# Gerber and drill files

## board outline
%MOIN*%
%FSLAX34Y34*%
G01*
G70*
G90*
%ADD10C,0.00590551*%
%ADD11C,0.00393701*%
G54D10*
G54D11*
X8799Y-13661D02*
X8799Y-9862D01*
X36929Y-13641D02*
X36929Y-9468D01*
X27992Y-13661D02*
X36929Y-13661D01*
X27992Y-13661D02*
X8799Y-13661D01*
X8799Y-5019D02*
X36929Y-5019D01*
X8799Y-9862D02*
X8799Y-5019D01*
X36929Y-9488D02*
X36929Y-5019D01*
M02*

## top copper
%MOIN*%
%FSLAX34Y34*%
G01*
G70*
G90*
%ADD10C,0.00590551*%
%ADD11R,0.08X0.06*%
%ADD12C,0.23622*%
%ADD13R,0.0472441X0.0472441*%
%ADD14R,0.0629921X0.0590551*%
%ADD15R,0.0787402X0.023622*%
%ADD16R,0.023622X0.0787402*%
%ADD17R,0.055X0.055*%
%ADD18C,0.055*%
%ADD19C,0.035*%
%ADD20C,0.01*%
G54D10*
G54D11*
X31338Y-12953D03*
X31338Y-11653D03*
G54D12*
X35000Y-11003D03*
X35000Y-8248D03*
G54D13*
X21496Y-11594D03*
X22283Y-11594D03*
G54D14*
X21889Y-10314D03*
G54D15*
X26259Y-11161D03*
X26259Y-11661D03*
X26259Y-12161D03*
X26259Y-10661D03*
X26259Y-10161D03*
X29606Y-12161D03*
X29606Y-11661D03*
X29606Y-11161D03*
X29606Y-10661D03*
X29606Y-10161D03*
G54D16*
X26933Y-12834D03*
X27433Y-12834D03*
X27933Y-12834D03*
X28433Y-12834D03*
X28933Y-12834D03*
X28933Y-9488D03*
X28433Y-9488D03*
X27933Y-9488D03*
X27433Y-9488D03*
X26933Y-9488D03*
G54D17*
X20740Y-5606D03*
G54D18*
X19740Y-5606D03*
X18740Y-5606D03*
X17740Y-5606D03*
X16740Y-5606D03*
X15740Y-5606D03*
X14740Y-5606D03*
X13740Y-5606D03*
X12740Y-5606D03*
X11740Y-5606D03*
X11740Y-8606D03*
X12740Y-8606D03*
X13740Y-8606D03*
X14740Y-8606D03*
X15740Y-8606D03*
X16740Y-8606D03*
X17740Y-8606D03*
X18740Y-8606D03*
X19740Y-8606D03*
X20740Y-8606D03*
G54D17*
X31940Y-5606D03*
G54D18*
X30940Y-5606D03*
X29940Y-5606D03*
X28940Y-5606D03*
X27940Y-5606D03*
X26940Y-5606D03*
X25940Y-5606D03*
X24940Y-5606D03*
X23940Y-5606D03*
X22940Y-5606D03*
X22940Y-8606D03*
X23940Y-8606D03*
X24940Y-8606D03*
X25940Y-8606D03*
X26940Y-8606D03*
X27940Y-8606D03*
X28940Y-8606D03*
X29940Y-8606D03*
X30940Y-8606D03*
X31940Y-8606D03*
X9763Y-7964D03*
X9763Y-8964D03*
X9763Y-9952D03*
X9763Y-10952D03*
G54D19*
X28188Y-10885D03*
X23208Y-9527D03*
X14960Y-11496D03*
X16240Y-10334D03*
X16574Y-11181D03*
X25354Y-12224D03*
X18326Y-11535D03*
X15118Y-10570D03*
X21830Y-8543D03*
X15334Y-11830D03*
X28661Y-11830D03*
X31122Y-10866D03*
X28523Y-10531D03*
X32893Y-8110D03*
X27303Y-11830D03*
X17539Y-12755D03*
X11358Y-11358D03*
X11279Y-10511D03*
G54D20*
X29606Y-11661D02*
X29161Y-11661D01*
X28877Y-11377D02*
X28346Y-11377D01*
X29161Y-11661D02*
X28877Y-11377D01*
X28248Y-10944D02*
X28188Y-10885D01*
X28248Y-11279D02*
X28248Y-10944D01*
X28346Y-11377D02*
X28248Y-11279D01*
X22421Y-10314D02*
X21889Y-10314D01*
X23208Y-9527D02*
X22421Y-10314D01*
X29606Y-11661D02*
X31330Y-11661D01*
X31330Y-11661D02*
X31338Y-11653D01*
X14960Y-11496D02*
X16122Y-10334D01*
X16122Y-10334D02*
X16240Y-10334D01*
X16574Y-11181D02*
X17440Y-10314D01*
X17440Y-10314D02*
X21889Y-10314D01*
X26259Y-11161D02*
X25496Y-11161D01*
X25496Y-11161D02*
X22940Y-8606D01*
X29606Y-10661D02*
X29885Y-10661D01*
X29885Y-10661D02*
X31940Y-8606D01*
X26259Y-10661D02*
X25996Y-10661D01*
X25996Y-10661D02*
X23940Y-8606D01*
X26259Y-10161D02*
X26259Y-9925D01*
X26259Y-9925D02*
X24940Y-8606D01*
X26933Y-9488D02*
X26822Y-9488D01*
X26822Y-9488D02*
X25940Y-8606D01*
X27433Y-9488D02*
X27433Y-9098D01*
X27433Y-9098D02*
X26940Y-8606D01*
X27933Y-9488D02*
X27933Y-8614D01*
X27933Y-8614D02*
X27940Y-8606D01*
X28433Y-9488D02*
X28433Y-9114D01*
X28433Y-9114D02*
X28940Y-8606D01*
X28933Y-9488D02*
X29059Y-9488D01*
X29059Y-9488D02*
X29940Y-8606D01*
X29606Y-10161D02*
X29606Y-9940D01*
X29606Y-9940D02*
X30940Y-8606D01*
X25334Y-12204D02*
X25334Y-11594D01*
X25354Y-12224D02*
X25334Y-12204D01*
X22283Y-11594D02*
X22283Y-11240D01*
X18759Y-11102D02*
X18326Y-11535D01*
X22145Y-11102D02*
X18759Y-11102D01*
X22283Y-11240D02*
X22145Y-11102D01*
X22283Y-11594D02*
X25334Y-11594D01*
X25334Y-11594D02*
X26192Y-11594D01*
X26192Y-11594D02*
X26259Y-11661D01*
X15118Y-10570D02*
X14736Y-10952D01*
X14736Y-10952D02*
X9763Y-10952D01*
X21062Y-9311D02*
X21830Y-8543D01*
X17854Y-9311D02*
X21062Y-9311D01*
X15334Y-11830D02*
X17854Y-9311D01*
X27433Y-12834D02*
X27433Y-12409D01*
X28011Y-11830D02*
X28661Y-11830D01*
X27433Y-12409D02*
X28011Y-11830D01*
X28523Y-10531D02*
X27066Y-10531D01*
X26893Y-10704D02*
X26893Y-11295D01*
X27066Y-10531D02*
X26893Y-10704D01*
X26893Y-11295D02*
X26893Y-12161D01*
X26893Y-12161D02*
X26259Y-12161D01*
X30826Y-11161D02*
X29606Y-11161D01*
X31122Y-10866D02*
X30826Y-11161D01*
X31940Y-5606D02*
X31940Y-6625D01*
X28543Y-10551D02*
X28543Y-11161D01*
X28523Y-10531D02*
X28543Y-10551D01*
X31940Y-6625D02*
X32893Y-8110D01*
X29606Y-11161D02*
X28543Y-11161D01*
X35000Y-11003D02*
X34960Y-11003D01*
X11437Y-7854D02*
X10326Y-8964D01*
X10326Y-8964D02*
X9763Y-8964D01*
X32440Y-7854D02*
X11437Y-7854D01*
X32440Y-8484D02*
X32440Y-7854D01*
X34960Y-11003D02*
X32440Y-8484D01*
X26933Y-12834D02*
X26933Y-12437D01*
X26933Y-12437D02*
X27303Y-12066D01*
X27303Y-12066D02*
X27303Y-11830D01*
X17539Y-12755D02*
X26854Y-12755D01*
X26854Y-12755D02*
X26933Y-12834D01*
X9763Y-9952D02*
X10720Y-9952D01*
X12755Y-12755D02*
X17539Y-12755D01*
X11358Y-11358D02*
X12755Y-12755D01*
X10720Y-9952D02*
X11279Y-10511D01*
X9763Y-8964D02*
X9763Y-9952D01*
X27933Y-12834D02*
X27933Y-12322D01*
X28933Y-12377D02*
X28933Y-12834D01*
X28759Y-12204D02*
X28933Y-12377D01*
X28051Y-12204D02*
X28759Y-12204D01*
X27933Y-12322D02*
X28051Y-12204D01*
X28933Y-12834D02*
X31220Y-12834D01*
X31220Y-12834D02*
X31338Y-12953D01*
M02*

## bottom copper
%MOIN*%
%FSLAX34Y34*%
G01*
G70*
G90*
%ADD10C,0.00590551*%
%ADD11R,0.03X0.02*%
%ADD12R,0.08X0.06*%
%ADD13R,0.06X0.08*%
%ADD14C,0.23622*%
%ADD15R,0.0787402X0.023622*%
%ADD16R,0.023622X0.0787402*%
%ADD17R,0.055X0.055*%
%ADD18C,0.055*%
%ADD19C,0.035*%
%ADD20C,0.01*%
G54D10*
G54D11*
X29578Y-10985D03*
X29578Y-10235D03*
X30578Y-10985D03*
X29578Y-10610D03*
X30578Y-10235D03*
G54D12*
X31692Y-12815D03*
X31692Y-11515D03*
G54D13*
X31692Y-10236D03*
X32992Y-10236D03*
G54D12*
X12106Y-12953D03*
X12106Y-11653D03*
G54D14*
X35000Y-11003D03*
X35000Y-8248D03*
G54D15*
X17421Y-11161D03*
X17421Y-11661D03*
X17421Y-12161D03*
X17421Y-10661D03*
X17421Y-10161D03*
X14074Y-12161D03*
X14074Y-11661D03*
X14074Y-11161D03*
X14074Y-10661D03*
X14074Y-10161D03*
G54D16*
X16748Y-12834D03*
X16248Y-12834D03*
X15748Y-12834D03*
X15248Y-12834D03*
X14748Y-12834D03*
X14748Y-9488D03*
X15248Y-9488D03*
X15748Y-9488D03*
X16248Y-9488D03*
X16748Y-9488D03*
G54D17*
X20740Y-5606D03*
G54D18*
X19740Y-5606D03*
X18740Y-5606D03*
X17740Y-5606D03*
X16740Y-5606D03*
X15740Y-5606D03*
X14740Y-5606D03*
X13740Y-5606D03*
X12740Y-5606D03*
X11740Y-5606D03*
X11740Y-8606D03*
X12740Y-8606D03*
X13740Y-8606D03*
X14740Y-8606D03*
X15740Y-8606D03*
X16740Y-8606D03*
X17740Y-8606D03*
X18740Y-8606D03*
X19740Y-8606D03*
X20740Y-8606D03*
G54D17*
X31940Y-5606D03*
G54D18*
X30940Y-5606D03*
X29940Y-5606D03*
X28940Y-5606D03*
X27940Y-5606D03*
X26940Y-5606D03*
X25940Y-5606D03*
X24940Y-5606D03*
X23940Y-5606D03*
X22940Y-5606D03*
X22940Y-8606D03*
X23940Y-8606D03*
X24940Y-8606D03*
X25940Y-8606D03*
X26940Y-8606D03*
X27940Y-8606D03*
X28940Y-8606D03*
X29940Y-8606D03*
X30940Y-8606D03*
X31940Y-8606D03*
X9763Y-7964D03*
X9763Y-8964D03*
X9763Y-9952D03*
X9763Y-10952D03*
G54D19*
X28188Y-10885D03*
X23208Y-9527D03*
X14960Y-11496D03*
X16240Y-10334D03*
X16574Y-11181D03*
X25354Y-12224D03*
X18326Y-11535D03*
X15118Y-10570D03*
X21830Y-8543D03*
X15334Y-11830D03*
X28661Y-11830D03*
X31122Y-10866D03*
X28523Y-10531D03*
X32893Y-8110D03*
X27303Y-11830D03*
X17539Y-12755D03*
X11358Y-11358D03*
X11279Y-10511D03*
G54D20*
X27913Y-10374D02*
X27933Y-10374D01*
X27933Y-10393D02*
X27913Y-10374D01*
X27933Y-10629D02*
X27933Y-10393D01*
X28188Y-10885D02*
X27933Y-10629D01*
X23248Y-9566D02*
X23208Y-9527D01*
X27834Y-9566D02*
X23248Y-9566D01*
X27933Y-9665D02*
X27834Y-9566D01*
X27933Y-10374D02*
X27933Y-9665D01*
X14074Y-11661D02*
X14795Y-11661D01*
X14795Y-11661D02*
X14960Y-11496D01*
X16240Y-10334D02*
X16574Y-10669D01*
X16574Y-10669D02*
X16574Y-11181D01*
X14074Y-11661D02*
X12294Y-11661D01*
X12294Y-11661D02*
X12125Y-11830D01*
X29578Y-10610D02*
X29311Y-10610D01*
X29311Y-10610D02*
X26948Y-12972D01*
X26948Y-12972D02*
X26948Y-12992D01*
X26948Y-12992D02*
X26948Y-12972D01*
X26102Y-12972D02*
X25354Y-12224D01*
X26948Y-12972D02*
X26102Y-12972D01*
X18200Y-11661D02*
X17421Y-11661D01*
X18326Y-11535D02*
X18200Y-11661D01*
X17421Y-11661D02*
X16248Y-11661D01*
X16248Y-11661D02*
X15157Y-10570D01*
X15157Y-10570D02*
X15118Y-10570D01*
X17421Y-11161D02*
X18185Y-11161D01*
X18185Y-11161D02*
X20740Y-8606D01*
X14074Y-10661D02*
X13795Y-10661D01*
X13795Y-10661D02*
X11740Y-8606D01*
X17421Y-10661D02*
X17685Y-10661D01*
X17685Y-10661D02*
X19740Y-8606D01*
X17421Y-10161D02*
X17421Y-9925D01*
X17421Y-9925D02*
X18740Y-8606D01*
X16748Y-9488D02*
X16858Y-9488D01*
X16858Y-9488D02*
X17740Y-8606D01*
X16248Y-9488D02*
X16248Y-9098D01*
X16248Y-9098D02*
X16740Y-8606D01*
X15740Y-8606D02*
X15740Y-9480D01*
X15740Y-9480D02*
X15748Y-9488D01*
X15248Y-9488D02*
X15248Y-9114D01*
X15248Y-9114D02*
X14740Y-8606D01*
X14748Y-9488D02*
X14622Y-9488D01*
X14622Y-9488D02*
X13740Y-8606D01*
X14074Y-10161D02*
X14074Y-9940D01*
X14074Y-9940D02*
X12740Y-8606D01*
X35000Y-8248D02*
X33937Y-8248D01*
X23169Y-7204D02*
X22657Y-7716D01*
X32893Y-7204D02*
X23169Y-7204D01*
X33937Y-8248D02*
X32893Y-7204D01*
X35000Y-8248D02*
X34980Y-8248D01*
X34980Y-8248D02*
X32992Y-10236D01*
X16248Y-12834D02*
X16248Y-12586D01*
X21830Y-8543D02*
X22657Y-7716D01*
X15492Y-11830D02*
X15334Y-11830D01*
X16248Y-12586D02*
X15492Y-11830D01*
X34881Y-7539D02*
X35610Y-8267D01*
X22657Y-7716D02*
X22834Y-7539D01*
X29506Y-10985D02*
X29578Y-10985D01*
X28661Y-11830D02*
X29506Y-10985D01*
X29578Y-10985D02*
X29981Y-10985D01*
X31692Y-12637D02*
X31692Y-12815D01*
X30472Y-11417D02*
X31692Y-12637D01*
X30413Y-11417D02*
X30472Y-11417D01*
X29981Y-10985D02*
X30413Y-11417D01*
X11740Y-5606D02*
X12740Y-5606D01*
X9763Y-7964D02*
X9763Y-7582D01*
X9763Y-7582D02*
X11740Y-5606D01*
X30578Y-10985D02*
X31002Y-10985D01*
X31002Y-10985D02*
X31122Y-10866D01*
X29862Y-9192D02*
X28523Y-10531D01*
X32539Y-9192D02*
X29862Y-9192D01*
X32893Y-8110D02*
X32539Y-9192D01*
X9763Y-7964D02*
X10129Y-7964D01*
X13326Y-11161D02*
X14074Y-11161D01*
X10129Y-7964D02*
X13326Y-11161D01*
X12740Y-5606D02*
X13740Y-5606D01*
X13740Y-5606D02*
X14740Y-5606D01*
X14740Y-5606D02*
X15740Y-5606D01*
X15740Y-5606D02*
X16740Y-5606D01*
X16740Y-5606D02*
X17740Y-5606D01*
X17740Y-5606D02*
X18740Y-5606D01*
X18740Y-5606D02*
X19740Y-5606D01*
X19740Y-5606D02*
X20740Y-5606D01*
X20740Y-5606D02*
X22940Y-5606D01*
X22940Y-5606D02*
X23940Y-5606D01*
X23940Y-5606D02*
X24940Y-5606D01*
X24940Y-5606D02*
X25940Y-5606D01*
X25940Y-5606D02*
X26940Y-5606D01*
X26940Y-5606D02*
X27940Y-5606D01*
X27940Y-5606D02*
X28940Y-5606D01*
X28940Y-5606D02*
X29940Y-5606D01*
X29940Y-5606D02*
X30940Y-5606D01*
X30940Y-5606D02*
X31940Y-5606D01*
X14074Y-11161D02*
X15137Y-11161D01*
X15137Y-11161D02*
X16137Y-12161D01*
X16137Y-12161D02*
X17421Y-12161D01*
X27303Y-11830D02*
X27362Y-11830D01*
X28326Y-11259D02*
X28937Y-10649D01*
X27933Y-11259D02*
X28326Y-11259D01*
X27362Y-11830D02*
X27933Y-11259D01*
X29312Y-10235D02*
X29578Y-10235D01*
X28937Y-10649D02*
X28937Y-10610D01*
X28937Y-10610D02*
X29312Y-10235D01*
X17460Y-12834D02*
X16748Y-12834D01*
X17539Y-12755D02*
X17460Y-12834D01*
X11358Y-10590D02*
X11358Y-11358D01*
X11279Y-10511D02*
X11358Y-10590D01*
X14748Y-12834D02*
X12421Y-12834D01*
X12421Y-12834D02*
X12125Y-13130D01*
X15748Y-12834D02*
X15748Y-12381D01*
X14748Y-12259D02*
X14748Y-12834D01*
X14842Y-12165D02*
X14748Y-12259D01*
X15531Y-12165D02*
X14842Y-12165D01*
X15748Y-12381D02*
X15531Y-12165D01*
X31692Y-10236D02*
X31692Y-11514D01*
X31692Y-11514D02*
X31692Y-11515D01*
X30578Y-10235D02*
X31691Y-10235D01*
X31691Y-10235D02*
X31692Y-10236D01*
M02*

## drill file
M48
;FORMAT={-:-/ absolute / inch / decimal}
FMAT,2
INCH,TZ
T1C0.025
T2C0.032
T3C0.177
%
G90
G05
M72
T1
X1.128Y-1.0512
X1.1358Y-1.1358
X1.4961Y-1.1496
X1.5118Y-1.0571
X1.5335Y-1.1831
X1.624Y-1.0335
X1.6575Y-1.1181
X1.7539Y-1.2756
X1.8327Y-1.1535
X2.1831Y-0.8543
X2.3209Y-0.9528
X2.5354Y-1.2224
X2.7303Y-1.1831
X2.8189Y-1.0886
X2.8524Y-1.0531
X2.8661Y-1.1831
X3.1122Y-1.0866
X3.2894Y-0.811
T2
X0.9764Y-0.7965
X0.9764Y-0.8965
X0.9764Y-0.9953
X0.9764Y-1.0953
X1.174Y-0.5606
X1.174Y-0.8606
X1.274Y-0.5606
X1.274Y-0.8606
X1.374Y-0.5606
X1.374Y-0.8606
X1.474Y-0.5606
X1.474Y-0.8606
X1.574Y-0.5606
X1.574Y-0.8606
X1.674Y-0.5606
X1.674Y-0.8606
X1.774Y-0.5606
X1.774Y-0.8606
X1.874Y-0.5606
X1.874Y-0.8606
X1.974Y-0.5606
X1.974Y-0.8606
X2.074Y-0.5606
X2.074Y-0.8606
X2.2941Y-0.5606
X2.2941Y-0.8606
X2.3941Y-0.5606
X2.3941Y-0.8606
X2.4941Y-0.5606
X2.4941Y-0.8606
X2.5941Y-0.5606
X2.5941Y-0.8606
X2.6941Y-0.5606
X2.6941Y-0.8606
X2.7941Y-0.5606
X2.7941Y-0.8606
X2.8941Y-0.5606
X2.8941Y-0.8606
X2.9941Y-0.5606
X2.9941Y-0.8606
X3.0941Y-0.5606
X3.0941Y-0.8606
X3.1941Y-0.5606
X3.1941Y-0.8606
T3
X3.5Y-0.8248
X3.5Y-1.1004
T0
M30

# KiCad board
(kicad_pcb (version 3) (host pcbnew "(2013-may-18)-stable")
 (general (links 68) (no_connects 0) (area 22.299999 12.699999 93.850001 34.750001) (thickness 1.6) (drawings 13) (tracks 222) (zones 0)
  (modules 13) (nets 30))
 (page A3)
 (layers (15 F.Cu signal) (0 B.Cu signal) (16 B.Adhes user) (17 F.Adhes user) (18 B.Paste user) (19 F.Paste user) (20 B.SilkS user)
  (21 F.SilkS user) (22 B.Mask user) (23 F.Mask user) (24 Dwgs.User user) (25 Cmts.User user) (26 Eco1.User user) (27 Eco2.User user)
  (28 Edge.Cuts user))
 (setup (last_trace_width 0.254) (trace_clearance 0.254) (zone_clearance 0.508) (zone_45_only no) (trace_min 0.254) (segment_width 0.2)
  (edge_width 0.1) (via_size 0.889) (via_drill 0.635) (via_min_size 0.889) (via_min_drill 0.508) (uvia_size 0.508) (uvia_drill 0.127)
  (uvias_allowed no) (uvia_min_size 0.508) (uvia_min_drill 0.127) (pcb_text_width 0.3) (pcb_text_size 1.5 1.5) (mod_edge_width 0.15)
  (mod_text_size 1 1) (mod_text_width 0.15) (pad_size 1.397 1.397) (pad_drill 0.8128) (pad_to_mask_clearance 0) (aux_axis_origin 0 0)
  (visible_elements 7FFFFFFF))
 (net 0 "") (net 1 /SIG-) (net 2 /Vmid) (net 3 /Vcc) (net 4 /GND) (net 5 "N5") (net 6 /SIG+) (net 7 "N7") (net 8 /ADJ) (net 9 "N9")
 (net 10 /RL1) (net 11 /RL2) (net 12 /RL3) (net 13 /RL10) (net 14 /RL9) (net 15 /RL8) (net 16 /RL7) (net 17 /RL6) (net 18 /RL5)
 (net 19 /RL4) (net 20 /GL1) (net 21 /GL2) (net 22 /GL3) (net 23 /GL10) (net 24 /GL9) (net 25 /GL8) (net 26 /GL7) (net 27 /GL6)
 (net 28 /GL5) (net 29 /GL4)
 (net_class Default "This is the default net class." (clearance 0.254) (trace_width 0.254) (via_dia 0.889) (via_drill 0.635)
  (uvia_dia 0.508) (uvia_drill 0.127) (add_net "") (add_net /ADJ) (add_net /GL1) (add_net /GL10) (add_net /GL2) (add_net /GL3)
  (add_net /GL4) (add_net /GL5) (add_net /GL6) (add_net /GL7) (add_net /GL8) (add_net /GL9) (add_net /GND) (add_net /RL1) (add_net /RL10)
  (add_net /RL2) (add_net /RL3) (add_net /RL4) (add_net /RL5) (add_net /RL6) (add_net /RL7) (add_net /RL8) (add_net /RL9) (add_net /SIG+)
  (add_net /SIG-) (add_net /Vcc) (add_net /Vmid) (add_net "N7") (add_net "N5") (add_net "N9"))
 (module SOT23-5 (layer B.Cu) (at 76.4 26.95 90)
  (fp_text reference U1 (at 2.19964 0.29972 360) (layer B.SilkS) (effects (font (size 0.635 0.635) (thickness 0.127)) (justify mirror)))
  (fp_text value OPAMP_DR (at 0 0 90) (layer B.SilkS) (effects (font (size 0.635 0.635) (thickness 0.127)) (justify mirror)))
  (pad 1 smd rect (at -0.9525 -1.27 90) (size 0.508 0.762) (layers B.Cu B.Paste B.Mask) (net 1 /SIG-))
  (pad 3 smd rect (at 0.9525 -1.27 90) (size 0.508 0.762) (layers B.Cu B.Paste B.Mask) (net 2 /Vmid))
  (pad 5 smd rect (at -0.9525 1.27 90) (size 0.508 0.762) (layers B.Cu B.Paste B.Mask) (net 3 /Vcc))
  (pad 2 smd rect (at 0 -1.27 90) (size 0.508 0.762) (layers B.Cu B.Paste B.Mask) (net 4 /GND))
  (pad 4 smd rect (at 0.9525 1.27 90) (size 0.508 0.762) (layers B.Cu B.Paste B.Mask) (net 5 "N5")))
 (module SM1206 (layer B.Cu) (at 80.5 30.9 90)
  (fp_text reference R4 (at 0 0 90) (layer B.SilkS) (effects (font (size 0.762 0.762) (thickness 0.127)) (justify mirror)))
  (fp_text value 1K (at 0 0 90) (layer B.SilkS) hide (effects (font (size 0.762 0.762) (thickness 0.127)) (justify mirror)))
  (pad 1 smd rect (at -1.651 0 90) (size 1.524 2.032) (layers B.Cu B.Paste B.Mask) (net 1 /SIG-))
  (pad 2 smd rect (at 1.651 0 90) (size 1.524 2.032) (layers B.Cu B.Paste B.Mask) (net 5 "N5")))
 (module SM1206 (layer B.Cu) (at 82.15 26)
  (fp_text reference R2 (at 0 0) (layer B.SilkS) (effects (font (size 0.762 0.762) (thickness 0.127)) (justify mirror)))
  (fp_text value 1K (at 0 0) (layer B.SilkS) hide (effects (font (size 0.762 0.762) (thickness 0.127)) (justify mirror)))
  (pad 1 smd rect (at -1.651 0) (size 1.524 2.032) (layers B.Cu B.Paste B.Mask) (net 5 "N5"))
  (pad 2 smd rect (at 1.651 0) (size 1.524 2.032) (layers B.Cu B.Paste B.Mask) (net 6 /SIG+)))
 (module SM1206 (layer B.Cu) (at 30.75 31.25 90)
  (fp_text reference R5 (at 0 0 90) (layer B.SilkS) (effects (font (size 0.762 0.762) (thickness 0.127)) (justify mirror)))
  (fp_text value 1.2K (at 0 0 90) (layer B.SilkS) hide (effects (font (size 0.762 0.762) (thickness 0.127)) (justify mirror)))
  (pad 1 smd rect (at -1.651 0 90) (size 1.524 2.032) (layers B.Cu B.Paste B.Mask) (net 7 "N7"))
  (pad 2 smd rect (at 1.651 0 90) (size 1.524 2.032) (layers B.Cu B.Paste B.Mask) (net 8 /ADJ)))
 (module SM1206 (layer F.Cu) (at 79.6 31.25 90)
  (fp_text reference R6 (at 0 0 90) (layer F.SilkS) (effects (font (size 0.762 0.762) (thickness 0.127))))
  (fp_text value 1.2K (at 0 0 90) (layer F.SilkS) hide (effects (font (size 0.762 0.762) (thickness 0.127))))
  (pad 1 smd rect (at -1.651 0 90) (size 1.524 2.032) (layers F.Cu F.Paste F.Mask) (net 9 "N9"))
  (pad 2 smd rect (at 1.651 0 90) (size 1.524 2.032) (layers F.Cu F.Paste F.Mask) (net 8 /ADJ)))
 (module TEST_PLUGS (layer F.Cu) (at 88.9 27.95 90)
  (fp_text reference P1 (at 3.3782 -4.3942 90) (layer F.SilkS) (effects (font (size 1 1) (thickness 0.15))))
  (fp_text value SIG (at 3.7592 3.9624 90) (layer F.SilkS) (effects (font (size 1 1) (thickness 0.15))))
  (pad 1 thru_hole circle (at 0 0 90) (size 6 6) (drill 4.5) (layers *.Cu *.Mask F.SilkS) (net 2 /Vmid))
  (pad 2 thru_hole circle (at 7 0 90) (size 6 6) (drill 4.5) (layers *.Cu *.Mask F.SilkS) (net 6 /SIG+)))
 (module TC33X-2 (layer F.Cu) (at 55.6 27.65)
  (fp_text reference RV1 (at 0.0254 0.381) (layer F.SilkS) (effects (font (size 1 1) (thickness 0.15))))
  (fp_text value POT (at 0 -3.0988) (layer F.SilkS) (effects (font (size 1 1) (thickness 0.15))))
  (pad 1 smd rect (at -1 1.8) (size 1.2 1.2) (layers F.Cu F.Paste F.Mask))
  (pad 3 smd rect (at 1 1.8) (size 1.2 1.2) (layers F.Cu F.Paste F.Mask) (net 4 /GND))
  (pad 2 smd rect (at 0 -1.45) (size 1.6 1.5) (layers F.Cu F.Paste F.Mask) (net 8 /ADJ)))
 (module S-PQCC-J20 (layer B.Cu) (at 40 28.35 90)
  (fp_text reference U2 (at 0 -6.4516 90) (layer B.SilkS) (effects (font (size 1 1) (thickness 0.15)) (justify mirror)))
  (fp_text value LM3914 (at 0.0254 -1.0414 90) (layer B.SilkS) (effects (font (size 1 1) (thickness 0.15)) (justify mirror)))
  (pad 1 smd rect (at 0 4.25 90) (size 0.6 2) (layers B.Cu B.Paste B.Mask) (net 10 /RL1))
  (pad 2 smd rect (at -1.27 4.25 90) (size 0.6 2) (layers B.Cu B.Paste B.Mask) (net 4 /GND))
  (pad 3 smd rect (at -2.54 4.25 90) (size 0.6 2) (layers B.Cu B.Paste B.Mask) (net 3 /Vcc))
  (pad 20 smd rect (at 1.27 4.25 90) (size 0.6 2) (layers B.Cu B.Paste B.Mask) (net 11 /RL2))
  (pad 19 smd rect (at 2.54 4.25 90) (size 0.6 2) (layers B.Cu B.Paste B.Mask) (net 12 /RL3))
  (pad 9 smd rect (at -2.54 -4.25 90) (size 0.6 2) (layers B.Cu B.Paste B.Mask))
  (pad 10 smd rect (at -1.27 -4.25 90) (size 0.6 2) (layers B.Cu B.Paste B.Mask) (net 8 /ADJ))
  (pad 11 smd rect (at 0 -4.25 90) (size 0.6 2) (layers B.Cu B.Paste B.Mask) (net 3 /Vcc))
  (pad 12 smd rect (at 1.27 -4.25 90) (size 0.6 2) (layers B.Cu B.Paste B.Mask) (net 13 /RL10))
  (pad 13 smd rect (at 2.54 -4.25 90) (size 0.6 2) (layers B.Cu B.Paste B.Mask) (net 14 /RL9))
  (pad 4 smd rect (at -4.25 2.54 90) (size 2 0.6) (layers B.Cu B.Paste B.Mask) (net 2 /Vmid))
  (pad 5 smd rect (at -4.25 1.27 90) (size 2 0.6) (layers B.Cu B.Paste B.Mask) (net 6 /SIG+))
  (pad 6 smd rect (at -4.25 0 90) (size 2 0.6) (layers B.Cu B.Paste B.Mask) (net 7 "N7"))
  (pad 7 smd rect (at -4.25 -1.27 90) (size 2 0.6) (layers B.Cu B.Paste B.Mask))
  (pad 8 smd rect (at -4.25 -2.54 90) (size 2 0.6) (layers B.Cu B.Paste B.Mask) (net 7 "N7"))
  (pad 14 smd rect (at 4.25 -2.54 90) (size 2 0.6) (layers B.Cu B.Paste B.Mask) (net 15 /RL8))
  (pad 15 smd rect (at 4.25 -1.27 90) (size 2 0.6) (layers B.Cu B.Paste B.Mask) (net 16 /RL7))
  (pad 16 smd rect (at 4.25 0 90) (size 2 0.6) (layers B.Cu B.Paste B.Mask) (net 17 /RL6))
  (pad 17 smd rect (at 4.25 1.27 90) (size 2 0.6) (layers B.Cu B.Paste B.Mask) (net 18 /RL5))
  (pad 18 smd rect (at 4.25 2.54 90) (size 2 0.6) (layers B.Cu B.Paste B.Mask) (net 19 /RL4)))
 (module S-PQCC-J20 (layer F.Cu) (at 70.95 28.35 90)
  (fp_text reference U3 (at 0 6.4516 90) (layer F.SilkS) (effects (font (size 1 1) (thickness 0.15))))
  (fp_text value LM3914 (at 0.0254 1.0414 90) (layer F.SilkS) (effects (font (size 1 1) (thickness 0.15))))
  (pad 1 smd rect (at 0 -4.25 90) (size 0.6 2) (layers F.Cu F.Paste F.Mask) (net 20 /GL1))
  (pad 2 smd rect (at -1.27 -4.25 90) (size 0.6 2) (layers F.Cu F.Paste F.Mask) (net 4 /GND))
  (pad 3 smd rect (at -2.54 -4.25 90) (size 0.6 2) (layers F.Cu F.Paste F.Mask) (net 3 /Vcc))
  (pad 20 smd rect (at 1.27 -4.25 90) (size 0.6 2) (layers F.Cu F.Paste F.Mask) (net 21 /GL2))
  (pad 19 smd rect (at 2.54 -4.25 90) (size 0.6 2) (layers F.Cu F.Paste F.Mask) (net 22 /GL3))
  (pad 9 smd rect (at -2.54 4.25 90) (size 0.6 2) (layers F.Cu F.Paste F.Mask))
  (pad 10 smd rect (at -1.27 4.25 90) (size 0.6 2) (layers F.Cu F.Paste F.Mask) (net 8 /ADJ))
  (pad 11 smd rect (at 0 4.25 90) (size 0.6 2) (layers F.Cu F.Paste F.Mask) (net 3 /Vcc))
  (pad 12 smd rect (at 1.27 4.25 90) (size 0.6 2) (layers F.Cu F.Paste F.Mask) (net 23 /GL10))
  (pad 13 smd rect (at 2.54 4.25 90) (size 0.6 2) (layers F.Cu F.Paste F.Mask) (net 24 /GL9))
  (pad 4 smd rect (at -4.25 -2.54 90) (size 2 0.6) (layers F.Cu F.Paste F.Mask) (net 2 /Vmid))
  (pad 5 smd rect (at -4.25 -1.27 90) (size 2 0.6) (layers F.Cu F.Paste F.Mask) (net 1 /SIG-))
  (pad 6 smd rect (at -4.25 0 90) (size 2 0.6) (layers F.Cu F.Paste F.Mask) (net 9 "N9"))
  (pad 7 smd rect (at -4.25 1.27 90) (size 2 0.6) (layers F.Cu F.Paste F.Mask))
  (pad 8 smd rect (at -4.25 2.54 90) (size 2 0.6) (layers F.Cu F.Paste F.Mask) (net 9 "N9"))
  (pad 14 smd rect (at 4.25 2.54 90) (size 2 0.6) (layers F.Cu F.Paste F.Mask) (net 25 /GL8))
  (pad 15 smd rect (at 4.25 1.27 90) (size 2 0.6) (layers F.Cu F.Paste F.Mask) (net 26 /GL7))
  (pad 16 smd rect (at 4.25 0 90) (size 2 0.6) (layers F.Cu F.Paste F.Mask) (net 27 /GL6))
  (pad 17 smd rect (at 4.25 -1.27 90) (size 2 0.6) (layers F.Cu F.Paste F.Mask) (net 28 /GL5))
  (pad 18 smd rect (at 4.25 -2.54 90) (size 2 0.6) (layers F.Cu F.Paste F.Mask) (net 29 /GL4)))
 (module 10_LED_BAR (layer F.Cu) (at 41.25 18.05 180)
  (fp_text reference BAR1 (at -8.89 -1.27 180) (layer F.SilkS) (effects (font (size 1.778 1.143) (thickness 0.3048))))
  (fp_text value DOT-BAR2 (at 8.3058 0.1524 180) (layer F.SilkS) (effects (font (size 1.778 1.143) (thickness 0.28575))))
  (pad 1 thru_hole rect (at -11.43 3.81 180) (size 1.397 1.397) (drill 0.8128) (layers *.Cu *.Mask F.SilkS) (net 3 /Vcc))
  (pad 2 thru_hole circle (at -8.89 3.81 180) (size 1.397 1.397) (drill 0.8128) (layers *.Cu *.Mask F.SilkS) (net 3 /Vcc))
  (pad 3 thru_hole circle (at -6.35 3.81 180) (size 1.397 1.397) (drill 0.8128) (layers *.Cu *.Mask F.SilkS) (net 3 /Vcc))
  (pad 4 thru_hole circle (at -3.81 3.81 180) (size 1.397 1.397) (drill 0.8128) (layers *.Cu *.Mask F.SilkS) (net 3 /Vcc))
  (pad 5 thru_hole circle (at -1.27 3.81 180) (size 1.397 1.397) (drill 0.8128) (layers *.Cu *.Mask F.SilkS) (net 3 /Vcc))
  (pad 6 thru_hole circle (at 1.27 3.81 180) (size 1.397 1.397) (drill 0.8128) (layers *.Cu *.Mask F.SilkS) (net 3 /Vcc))
  (pad 7 thru_hole circle (at 3.81 3.81 180) (size 1.397 1.397) (drill 0.8128) (layers *.Cu *.Mask F.SilkS) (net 3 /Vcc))
  (pad 8 thru_hole circle (at 6.35 3.81 180) (size 1.397 1.397) (drill 0.8128) (layers *.Cu *.Mask F.SilkS) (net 3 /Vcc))
  (pad 9 thru_hole circle (at 8.89 3.81 180) (size 1.397 1.397) (drill 0.8128) (layers *.Cu *.Mask F.SilkS) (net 3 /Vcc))
  (pad 10 thru_hole circle (at 11.43 3.81 180) (size 1.397 1.397) (drill 0.8128) (layers *.Cu *.Mask F.SilkS) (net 3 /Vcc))
  (pad 11 thru_hole circle (at 11.43 -3.81 180) (size 1.397 1.397) (drill 0.8128) (layers *.Cu *.Mask F.SilkS) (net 13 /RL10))
  (pad 12 thru_hole circle (at 8.89 -3.81 180) (size 1.397 1.397) (drill 0.8128) (layers *.Cu *.Mask F.SilkS) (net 14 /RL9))
  (pad 13 thru_hole circle (at 6.35 -3.81 180) (size 1.397 1.397) (drill 0.8128) (layers *.Cu *.Mask F.SilkS) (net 15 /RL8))
  (pad 14 thru_hole circle (at 3.81 -3.81 180) (size 1.397 1.397) (drill 0.8128) (layers *.Cu *.Mask F.SilkS) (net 16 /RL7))
  (pad 15 thru_hole circle (at 1.27 -3.81 180) (size 1.397 1.397) (drill 0.8128) (layers *.Cu *.Mask F.SilkS) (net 17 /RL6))
  (pad 16 thru_hole circle (at -1.27 -3.81 180) (size 1.397 1.397) (drill 0.8128) (layers *.Cu *.Mask F.SilkS) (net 18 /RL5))
  (pad 17 thru_hole circle (at -3.81 -3.81 180) (size 1.397 1.397) (drill 0.8128) (layers *.Cu *.Mask F.SilkS) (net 19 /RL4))
  (pad 18 thru_hole circle (at -6.35 -3.81 180) (size 1.397 1.397) (drill 0.8128) (layers *.Cu *.Mask F.SilkS) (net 12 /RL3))
  (pad 19 thru_hole circle (at -8.89 -3.81 180) (size 1.397 1.397) (drill 0.8128) (layers *.Cu *.Mask F.SilkS) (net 11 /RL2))
  (pad 20 thru_hole circle (at -11.43 -3.81 180) (size 1.397 1.397) (drill 0.8128) (layers *.Cu *.Mask F.SilkS) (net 10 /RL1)))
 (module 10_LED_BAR (layer F.Cu) (at 69.7 18.05 180)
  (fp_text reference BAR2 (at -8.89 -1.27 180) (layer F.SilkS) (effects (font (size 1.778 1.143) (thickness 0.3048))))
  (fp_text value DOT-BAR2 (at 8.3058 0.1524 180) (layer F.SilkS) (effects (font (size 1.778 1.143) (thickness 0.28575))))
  (pad 1 thru_hole rect (at -11.43 3.81 180) (size 1.397 1.397) (drill 0.8128) (layers *.Cu *.Mask F.SilkS) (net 3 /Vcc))
  (pad 2 thru_hole circle (at -8.89 3.81 180) (size 1.397 1.397) (drill 0.8128) (layers *.Cu *.Mask F.SilkS) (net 3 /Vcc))
  (pad 3 thru_hole circle (at -6.35 3.81 180) (size 1.397 1.397) (drill 0.8128) (layers *.Cu *.Mask F.SilkS) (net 3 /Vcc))
  (pad 4 thru_hole circle (at -3.81 3.81 180) (size 1.397 1.397) (drill 0.8128) (layers *.Cu *.Mask F.SilkS) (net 3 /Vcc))
  (pad 5 thru_hole circle (at -1.27 3.81 180) (size 1.397 1.397) (drill 0.8128) (layers *.Cu *.Mask F.SilkS) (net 3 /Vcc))
  (pad 6 thru_hole circle (at 1.27 3.81 180) (size 1.397 1.397) (drill 0.8128) (layers *.Cu *.Mask F.SilkS) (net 3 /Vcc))
  (pad 7 thru_hole circle (at 3.81 3.81 180) (size 1.397 1.397) (drill 0.8128) (layers *.Cu *.Mask F.SilkS) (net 3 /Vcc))
  (pad 8 thru_hole circle (at 6.35 3.81 180) (size 1.397 1.397) (drill 0.8128) (layers *.Cu *.Mask F.SilkS) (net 3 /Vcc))
  (pad 9 thru_hole circle (at 8.89 3.81 180) (size 1.397 1.397) (drill 0.8128) (layers *.Cu *.Mask F.SilkS) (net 3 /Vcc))
  (pad 10 thru_hole circle (at 11.43 3.81 180) (size 1.397 1.397) (drill 0.8128) (layers *.Cu *.Mask F.SilkS) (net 3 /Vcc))
  (pad 11 thru_hole circle (at 11.43 -3.81 180) (size 1.397 1.397) (drill 0.8128) (layers *.Cu *.Mask F.SilkS) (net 20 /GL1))
  (pad 12 thru_hole circle (at 8.89 -3.81 180) (size 1.397 1.397) (drill 0.8128) (layers *.Cu *.Mask F.SilkS) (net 21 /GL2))
  (pad 13 thru_hole circle (at 6.35 -3.81 180) (size 1.397 1.397) (drill 0.8128) (layers *.Cu *.Mask F.SilkS) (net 22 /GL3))
  (pad 14 thru_hole circle (at 3.81 -3.81 180) (size 1.397 1.397) (drill 0.8128) (layers *.Cu *.Mask F.SilkS) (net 29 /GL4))
  (pad 15 thru_hole circle (at 1.27 -3.81 180) (size 1.397 1.397) (drill 0.8128) (layers *.Cu *.Mask F.SilkS) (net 28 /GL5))
  (pad 16 thru_hole circle (at -1.27 -3.81 180) (size 1.397 1.397) (drill 0.8128) (layers *.Cu *.Mask F.SilkS) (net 27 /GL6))
  (pad 17 thru_hole circle (at -3.81 -3.81 180) (size 1.397 1.397) (drill 0.8128) (layers *.Cu *.Mask F.SilkS) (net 26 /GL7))
  (pad 18 thru_hole circle (at -6.35 -3.81 180) (size 1.397 1.397) (drill 0.8128) (layers *.Cu *.Mask F.SilkS) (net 25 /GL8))
  (pad 19 thru_hole circle (at -8.89 -3.81 180) (size 1.397 1.397) (drill 0.8128) (layers *.Cu *.Mask F.SilkS) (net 24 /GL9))
  (pad 20 thru_hole circle (at -11.43 -3.81 180) (size 1.397 1.397) (drill 0.8128) (layers *.Cu *.Mask F.SilkS) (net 23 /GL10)))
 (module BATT (layer F.Cu) (at 24.8 21.5 270)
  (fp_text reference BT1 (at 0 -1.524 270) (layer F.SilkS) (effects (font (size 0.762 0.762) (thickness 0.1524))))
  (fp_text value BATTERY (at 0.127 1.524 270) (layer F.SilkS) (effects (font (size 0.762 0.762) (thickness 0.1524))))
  (pad 1 thru_hole circle (at -1.27 0 270) (size 1.397 1.397) (drill 0.8128) (layers *.Cu *.Mask F.SilkS) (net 3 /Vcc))
  (pad 2 thru_hole circle (at 1.27 0 270) (size 1.397 1.397) (drill 0.8128) (layers *.Cu *.Mask F.SilkS) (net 2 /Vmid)))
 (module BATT (layer F.Cu) (at 24.8 26.55 270)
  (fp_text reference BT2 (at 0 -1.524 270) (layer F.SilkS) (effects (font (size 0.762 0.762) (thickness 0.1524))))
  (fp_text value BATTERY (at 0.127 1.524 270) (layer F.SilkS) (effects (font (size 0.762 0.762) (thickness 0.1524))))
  (pad 1 thru_hole circle (at -1.27 0 270) (size 1.397 1.397) (drill 0.8128) (layers *.Cu *.Mask F.SilkS) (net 2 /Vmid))
  (pad 2 thru_hole circle (at 1.27 0 270) (size 1.397 1.397) (drill 0.8128) (layers *.Cu *.Mask F.SilkS) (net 4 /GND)))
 (gr_line (start 22.35 34.7) (end 22.35 25.05) (angle 90) (layer Edge.Cuts) (width 0.1))
 (gr_line (start 93.8 34.65) (end 93.8 24.05) (angle 90) (layer Edge.Cuts) (width 0.1))
 (gr_line (start 71.1 34.7) (end 93.8 34.7) (angle 90) (layer Edge.Cuts) (width 0.1))
 (gr_line (start 71.1 34.7) (end 22.35 34.7) (angle 90) (layer Edge.Cuts) (width 0.1))
 (gr_line (start 22.35 12.75) (end 93.8 12.75) (angle 90) (layer Edge.Cuts) (width 0.1))
 (gr_line (start 22.35 25.05) (end 22.35 12.75) (angle 90) (layer Edge.Cuts) (width 0.1))
 (gr_line (start 93.8 24.1) (end 93.8 12.75) (angle 90) (layer Edge.Cuts) (width 0.1))
 (segment (start 75.2 29.62) (end 74.07 29.62) (width 0.254) (layer F.Cu) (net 8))
 (segment (start 73.35 28.9) (end 72 28.9) (width 0.254) (layer F.Cu) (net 8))
 (segment (start 74.07 29.62) (end 73.35 28.9) (width 0.254) (layer F.Cu) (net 8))
 (segment (start 70.9 26.35) (end 70.95 26.35) (width 0.254) (layer B.Cu) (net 8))
 (segment (start 70.95 26.4) (end 70.9 26.35) (width 0.254) (layer B.Cu) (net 8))
 (segment (start 70.95 27) (end 70.95 26.4) (width 0.254) (layer B.Cu) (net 8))
 (segment (start 71.6 27.65) (end 70.95 27) (width 0.254) (layer B.Cu) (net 8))
 (via (at 71.6 27.65) (size 0.889) (layers F.Cu B.Cu) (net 8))
 (segment (start 71.75 27.8) (end 71.6 27.65) (width 0.254) (layer F.Cu) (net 8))
 (segment (start 71.75 28.65) (end 71.75 27.8) (width 0.254) (layer F.Cu) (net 8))
 (segment (start 72 28.9) (end 71.75 28.65) (width 0.254) (layer F.Cu) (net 8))
 (segment (start 56.95 26.2) (end 55.6 26.2) (width 0.254) (layer F.Cu) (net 8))
 (segment (start 58.95 24.2) (end 56.95 26.2) (width 0.254) (layer F.Cu) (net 8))
 (via (at 58.95 24.2) (size 0.889) (layers F.Cu B.Cu) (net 8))
 (segment (start 59.05 24.3) (end 58.95 24.2) (width 0.254) (layer B.Cu) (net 8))
 (segment (start 70.7 24.3) (end 59.05 24.3) (width 0.254) (layer B.Cu) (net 8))
 (segment (start 70.95 24.55) (end 70.7 24.3) (width 0.254) (layer B.Cu) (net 8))
 (segment (start 70.95 26.35) (end 70.95 24.55) (width 0.254) (layer B.Cu) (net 8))
 (segment (start 75.2 29.62) (end 79.579 29.62) (width 0.254) (layer F.Cu) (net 8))
 (segment (start 79.579 29.62) (end 79.6 29.599) (width 0.254) (layer F.Cu) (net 8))
 (segment (start 35.75 29.62) (end 37.58 29.62) (width 0.254) (layer B.Cu) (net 8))
 (segment (start 37.58 29.62) (end 38 29.2) (width 0.254) (layer B.Cu) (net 8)) (via (at 38 29.2) (size 0.889) (layers F.Cu B.Cu) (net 8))
 (segment (start 38 29.2) (end 40.95 26.25) (width 0.254) (layer F.Cu) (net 8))
 (segment (start 40.95 26.25) (end 41.25 26.25) (width 0.254) (layer F.Cu) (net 8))
 (via (at 41.25 26.25) (size 0.889) (layers F.Cu B.Cu) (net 8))
 (segment (start 41.25 26.25) (end 42.1 27.1) (width 0.254) (layer B.Cu) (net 8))
 (segment (start 42.1 27.1) (end 42.1 28.4) (width 0.254) (layer B.Cu) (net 8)) (via (at 42.1 28.4) (size 0.889) (layers F.Cu B.Cu) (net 8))
 (segment (start 42.1 28.4) (end 44.3 26.2) (width 0.254) (layer F.Cu) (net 8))
 (segment (start 44.3 26.2) (end 55.6 26.2) (width 0.254) (layer F.Cu) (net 8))
 (segment (start 35.75 29.62) (end 31.229 29.62) (width 0.254) (layer B.Cu) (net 8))
 (segment (start 31.229 29.62) (end 30.8 30.049) (width 0.254) (layer B.Cu) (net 8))
 (segment (start 66.7 28.35) (end 64.76 28.35) (width 0.254) (layer F.Cu) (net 20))
 (segment (start 64.76 28.35) (end 58.27 21.86) (width 0.254) (layer F.Cu) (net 20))
 (segment (start 75.2 27.08) (end 75.91 27.08) (width 0.254) (layer F.Cu) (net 23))
 (segment (start 75.91 27.08) (end 81.13 21.86) (width 0.254) (layer F.Cu) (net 23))
 (segment (start 66.7 27.08) (end 66.03 27.08) (width 0.254) (layer F.Cu) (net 21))
 (segment (start 66.03 27.08) (end 60.81 21.86) (width 0.254) (layer F.Cu) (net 21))
 (segment (start 66.7 25.81) (end 66.7 25.21) (width 0.254) (layer F.Cu) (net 22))
 (segment (start 66.7 25.21) (end 63.35 21.86) (width 0.254) (layer F.Cu) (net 22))
 (segment (start 68.41 24.1) (end 68.13 24.1) (width 0.254) (layer F.Cu) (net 29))
 (segment (start 68.13 24.1) (end 65.89 21.86) (width 0.254) (layer F.Cu) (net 29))
 (segment (start 69.68 24.1) (end 69.68 23.11) (width 0.254) (layer F.Cu) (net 28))
 (segment (start 69.68 23.11) (end 68.43 21.86) (width 0.254) (layer F.Cu) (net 28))
 (segment (start 70.95 24.1) (end 70.95 21.88) (width 0.254) (layer F.Cu) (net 27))
 (segment (start 70.95 21.88) (end 70.97 21.86) (width 0.254) (layer F.Cu) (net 27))
 (segment (start 72.22 24.1) (end 72.22 23.15) (width 0.254) (layer F.Cu) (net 26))
 (segment (start 72.22 23.15) (end 73.51 21.86) (width 0.254) (layer F.Cu) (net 26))
 (segment (start 73.49 24.1) (end 73.81 24.1) (width 0.254) (layer F.Cu) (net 25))
 (segment (start 73.81 24.1) (end 76.05 21.86) (width 0.254) (layer F.Cu) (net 25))
 (segment (start 75.2 25.81) (end 75.2 25.25) (width 0.254) (layer F.Cu) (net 24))
 (segment (start 75.2 25.25) (end 78.59 21.86) (width 0.254) (layer F.Cu) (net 24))
 (segment (start 75.13 26.95) (end 74.45 26.95) (width 0.254) (layer B.Cu) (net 4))
 (segment (start 74.45 26.95) (end 68.45 32.95) (width 0.254) (layer B.Cu) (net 4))
 (segment (start 68.45 32.95) (end 68.45 33) (width 0.254) (layer B.Cu) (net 4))
 (segment (start 68.45 33) (end 68.45 32.95) (width 0.254) (layer B.Cu) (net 4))
 (segment (start 64.35 31) (end 64.35 29.45) (width 0.254) (layer F.Cu) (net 4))
 (segment (start 64.4 31.05) (end 64.35 31) (width 0.254) (layer F.Cu) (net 4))
 (via (at 64.4 31.05) (size 0.889) (layers F.Cu B.Cu) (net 4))
 (segment (start 66.3 32.95) (end 64.4 31.05) (width 0.254) (layer B.Cu) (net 4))
 (segment (start 68.45 32.95) (end 66.3 32.95) (width 0.254) (layer B.Cu) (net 4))
 (segment (start 56.6 29.45) (end 56.6 28.55) (width 0.254) (layer F.Cu) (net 4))
 (segment (start 46.23 29.62) (end 44.25 29.62) (width 0.254) (layer B.Cu) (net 4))
 (segment (start 46.55 29.3) (end 46.23 29.62) (width 0.254) (layer B.Cu) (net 4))
 (via (at 46.55 29.3) (size 0.889) (layers F.Cu B.Cu) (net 4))
 (segment (start 47.65 28.2) (end 46.55 29.3) (width 0.254) (layer F.Cu) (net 4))
 (segment (start 56.25 28.2) (end 47.65 28.2) (width 0.254) (layer F.Cu) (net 4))
 (segment (start 56.6 28.55) (end 56.25 28.2) (width 0.254) (layer F.Cu) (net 4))
 (segment (start 56.6 29.45) (end 64.35 29.45) (width 0.254) (layer F.Cu) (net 4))
 (segment (start 64.35 29.45) (end 66.53 29.45) (width 0.254) (layer F.Cu) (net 4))
 (segment (start 66.53 29.45) (end 66.7 29.62) (width 0.254) (layer F.Cu) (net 4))
 (segment (start 44.25 29.62) (end 41.27 29.62) (width 0.254) (layer B.Cu) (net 4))
 (segment (start 41.27 29.62) (end 38.5 26.85) (width 0.254) (layer B.Cu) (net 4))
 (segment (start 38.5 26.85) (end 38.4 26.85) (width 0.254) (layer B.Cu) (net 4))
 (via (at 38.4 26.85) (size 0.889) (layers F.Cu B.Cu) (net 4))
 (segment (start 38.4 26.85) (end 37.43 27.82) (width 0.254) (layer F.Cu) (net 4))
 (segment (start 37.43 27.82) (end 24.8 27.82) (width 0.254) (layer F.Cu) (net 4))
 (segment (start 44.25 28.35) (end 46.19 28.35) (width 0.254) (layer B.Cu) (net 10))
 (segment (start 46.19 28.35) (end 52.68 21.86) (width 0.254) (layer B.Cu) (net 10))
 (segment (start 35.75 27.08) (end 35.04 27.08) (width 0.254) (layer B.Cu) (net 13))
 (segment (start 35.04 27.08) (end 29.82 21.86) (width 0.254) (layer B.Cu) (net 13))
 (segment (start 44.25 27.08) (end 44.92 27.08) (width 0.254) (layer B.Cu) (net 11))
 (segment (start 44.92 27.08) (end 50.14 21.86) (width 0.254) (layer B.Cu) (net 11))
 (segment (start 44.25 25.81) (end 44.25 25.21) (width 0.254) (layer B.Cu) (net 12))
 (segment (start 44.25 25.21) (end 47.6 21.86) (width 0.254) (layer B.Cu) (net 12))
 (segment (start 42.54 24.1) (end 42.82 24.1) (width 0.254) (layer B.Cu) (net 19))
 (segment (start 42.82 24.1) (end 45.06 21.86) (width 0.254) (layer B.Cu) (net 19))
 (segment (start 41.27 24.1) (end 41.27 23.11) (width 0.254) (layer B.Cu) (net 18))
 (segment (start 41.27 23.11) (end 42.52 21.86) (width 0.254) (layer B.Cu) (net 18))
 (segment (start 39.98 21.86) (end 39.98 24.08) (width 0.254) (layer B.Cu) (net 17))
 (segment (start 39.98 24.08) (end 40 24.1) (width 0.254) (layer B.Cu) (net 17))
 (segment (start 38.73 24.1) (end 38.73 23.15) (width 0.254) (layer B.Cu) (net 16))
 (segment (start 38.73 23.15) (end 37.44 21.86) (width 0.254) (layer B.Cu) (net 16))
 (segment (start 37.46 24.1) (end 37.14 24.1) (width 0.254) (layer B.Cu) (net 15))
 (segment (start 37.14 24.1) (end 34.9 21.86) (width 0.254) (layer B.Cu) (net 15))
 (segment (start 35.75 25.81) (end 35.75 25.25) (width 0.254) (layer B.Cu) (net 14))
 (segment (start 35.75 25.25) (end 32.36 21.86) (width 0.254) (layer B.Cu) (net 14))
 (segment (start 88.9 20.95) (end 86.2 20.95) (width 0.254) (layer B.Cu) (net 6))
 (segment (start 58.85 18.3) (end 57.55 19.6) (width 0.254) (layer B.Cu) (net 6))
 (segment (start 83.55 18.3) (end 58.85 18.3) (width 0.254) (layer B.Cu) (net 6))
 (segment (start 86.2 20.95) (end 83.55 18.3) (width 0.254) (layer B.Cu) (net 6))
 (segment (start 88.9 20.95) (end 88.851 20.95) (width 0.254) (layer B.Cu) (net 6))
 (segment (start 88.851 20.95) (end 83.801 26) (width 0.254) (layer B.Cu) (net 6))
 (segment (start 41.27 32.6) (end 41.27 31.97) (width 0.254) (layer B.Cu) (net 6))
 (segment (start 55.45 21.7) (end 57.55 19.6) (width 0.254) (layer B.Cu) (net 6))
 (via (at 55.45 21.7) (size 0.889) (layers F.Cu B.Cu) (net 6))
 (segment (start 53.5 23.65) (end 55.45 21.7) (width 0.254) (layer F.Cu) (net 6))
 (segment (start 45.35 23.65) (end 53.5 23.65) (width 0.254) (layer F.Cu) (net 6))
 (segment (start 38.95 30.05) (end 45.35 23.65) (width 0.254) (layer F.Cu) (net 6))
 (via (at 38.95 30.05) (size 0.889) (layers F.Cu B.Cu) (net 6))
 (segment (start 39.35 30.05) (end 38.95 30.05) (width 0.254) (layer B.Cu) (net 6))
 (segment (start 41.27 31.97) (end 39.35 30.05) (width 0.254) (layer B.Cu) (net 6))
 (segment (start 88.6 19.15) (end 90.45 21) (width 0.254) (layer B.Cu) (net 6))
 (segment (start 57.55 19.6) (end 58 19.15) (width 0.254) (layer B.Cu) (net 6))
 (segment (start 69.68 32.6) (end 69.68 31.52) (width 0.254) (layer F.Cu) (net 1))
 (segment (start 74.9475 27.9025) (end 75.13 27.9025) (width 0.254) (layer B.Cu) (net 1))
 (segment (start 72.8 30.05) (end 74.9475 27.9025) (width 0.254) (layer B.Cu) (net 1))
 (via (at 72.8 30.05) (size 0.889) (layers F.Cu B.Cu) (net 1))
 (segment (start 71.15 30.05) (end 72.8 30.05) (width 0.254) (layer F.Cu) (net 1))
 (segment (start 69.68 31.52) (end 71.15 30.05) (width 0.254) (layer F.Cu) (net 1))
 (segment (start 75.13 27.9025) (end 76.1525 27.9025) (width 0.254) (layer B.Cu) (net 1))
 (segment (start 80.5 32.1) (end 80.5 32.551) (width 0.254) (layer B.Cu) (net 1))
 (segment (start 77.4 29) (end 80.5 32.1) (width 0.254) (layer B.Cu) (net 1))
 (segment (start 77.25 29) (end 77.4 29) (width 0.254) (layer B.Cu) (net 1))
 (segment (start 76.1525 27.9025) (end 77.25 29) (width 0.254) (layer B.Cu) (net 1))
 (segment (start 29.82 14.24) (end 32.36 14.24) (width 0.254) (layer B.Cu) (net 3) (status C00000))
 (segment (start 24.8 20.23) (end 24.8 19.26) (width 0.254) (layer B.Cu) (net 3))
 (segment (start 24.8 19.26) (end 29.82 14.24) (width 0.254) (layer B.Cu) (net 3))
 (segment (start 72.45 26.75) (end 68.75 26.75) (width 0.254) (layer F.Cu) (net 3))
 (segment (start 68.31 27.19) (end 68.31 28.69) (width 0.254) (layer F.Cu) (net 3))
 (segment (start 68.75 26.75) (end 68.31 27.19) (width 0.254) (layer F.Cu) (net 3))
 (segment (start 68.31 28.69) (end 68.31 30.89) (width 0.254) (layer F.Cu) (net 3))
 (segment (start 68.31 30.89) (end 66.7 30.89) (width 0.254) (layer F.Cu) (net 3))
 (segment (start 77.67 27.9025) (end 78.7475 27.9025) (width 0.254) (layer B.Cu) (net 3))
 (segment (start 78.3 28.35) (end 75.2 28.35) (width 0.254) (layer F.Cu) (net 3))
 (segment (start 79.05 27.6) (end 78.3 28.35) (width 0.254) (layer F.Cu) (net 3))
 (via (at 79.05 27.6) (size 0.889) (layers F.Cu B.Cu) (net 3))
 (segment (start 78.7475 27.9025) (end 79.05 27.6) (width 0.254) (layer B.Cu) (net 3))
 (segment (start 81.13 14.24) (end 81.13 16.83) (width 0.254) (layer F.Cu) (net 3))
 (segment (start 72.5 26.8) (end 72.5 28.35) (width 0.254) (layer F.Cu) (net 3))
 (segment (start 72.45 26.75) (end 72.5 26.8) (width 0.254) (layer F.Cu) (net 3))
 (via (at 72.45 26.75) (size 0.889) (layers F.Cu B.Cu) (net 3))
 (segment (start 75.85 23.35) (end 72.45 26.75) (width 0.254) (layer B.Cu) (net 3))
 (segment (start 82.65 23.35) (end 75.85 23.35) (width 0.254) (layer B.Cu) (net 3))
 (segment (start 83.55 20.6) (end 82.65 23.35) (width 0.254) (layer B.Cu) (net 3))
 (via (at 83.55 20.6) (size 0.889) (layers F.Cu B.Cu) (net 3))
 (segment (start 81.13 16.83) (end 83.55 20.6) (width 0.254) (layer F.Cu) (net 3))
 (segment (start 24.8 20.23) (end 25.73 20.23) (width 0.254) (layer B.Cu) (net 3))
 (segment (start 33.85 28.35) (end 35.75 28.35) (width 0.254) (layer B.Cu) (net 3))
 (segment (start 25.73 20.23) (end 33.85 28.35) (width 0.254) (layer B.Cu) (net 3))
 (segment (start 32.36 14.24) (end 34.9 14.24) (width 0.254) (layer B.Cu) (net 3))
 (segment (start 34.9 14.24) (end 37.44 14.24) (width 0.254) (layer B.Cu) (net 3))
 (segment (start 37.44 14.24) (end 39.98 14.24) (width 0.254) (layer B.Cu) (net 3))
 (segment (start 39.98 14.24) (end 42.52 14.24) (width 0.254) (layer B.Cu) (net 3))
 (segment (start 42.52 14.24) (end 45.06 14.24) (width 0.254) (layer B.Cu) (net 3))
 (segment (start 45.06 14.24) (end 47.6 14.24) (width 0.254) (layer B.Cu) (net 3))
 (segment (start 47.6 14.24) (end 50.14 14.24) (width 0.254) (layer B.Cu) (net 3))
 (segment (start 50.14 14.24) (end 52.68 14.24) (width 0.254) (layer B.Cu) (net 3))
 (segment (start 52.68 14.24) (end 58.27 14.24) (width 0.254) (layer B.Cu) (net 3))
 (segment (start 58.27 14.24) (end 60.81 14.24) (width 0.254) (layer B.Cu) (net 3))
 (segment (start 60.81 14.24) (end 63.35 14.24) (width 0.254) (layer B.Cu) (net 3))
 (segment (start 63.35 14.24) (end 65.89 14.24) (width 0.254) (layer B.Cu) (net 3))
 (segment (start 65.89 14.24) (end 68.43 14.24) (width 0.254) (layer B.Cu) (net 3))
 (segment (start 68.43 14.24) (end 70.97 14.24) (width 0.254) (layer B.Cu) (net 3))
 (segment (start 70.97 14.24) (end 73.51 14.24) (width 0.254) (layer B.Cu) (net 3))
 (segment (start 73.51 14.24) (end 76.05 14.24) (width 0.254) (layer B.Cu) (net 3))
 (segment (start 76.05 14.24) (end 78.59 14.24) (width 0.254) (layer B.Cu) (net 3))
 (segment (start 78.59 14.24) (end 81.13 14.24) (width 0.254) (layer B.Cu) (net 3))
 (segment (start 35.75 28.35) (end 38.45 28.35) (width 0.254) (layer B.Cu) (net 3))
 (segment (start 38.45 28.35) (end 40.99 30.89) (width 0.254) (layer B.Cu) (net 3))
 (segment (start 40.99 30.89) (end 44.25 30.89) (width 0.254) (layer B.Cu) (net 3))
 (segment (start 75.2 28.35) (end 72.5 28.35) (width 0.254) (layer F.Cu) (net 3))
 (segment (start 88.9 27.95) (end 88.8 27.95) (width 0.254) (layer F.Cu) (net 2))
 (segment (start 29.05 19.95) (end 26.23 22.77) (width 0.254) (layer F.Cu) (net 2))
 (segment (start 26.23 22.77) (end 24.8 22.77) (width 0.254) (layer F.Cu) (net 2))
 (segment (start 82.4 19.95) (end 29.05 19.95) (width 0.254) (layer F.Cu) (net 2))
 (segment (start 82.4 21.55) (end 82.4 19.95) (width 0.254) (layer F.Cu) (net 2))
 (segment (start 88.8 27.95) (end 82.4 21.55) (width 0.254) (layer F.Cu) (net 2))
 (segment (start 69.35 30.05) (end 69.5 30.05) (width 0.254) (layer B.Cu) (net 2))
 (segment (start 71.95 28.6) (end 73.5 27.05) (width 0.254) (layer B.Cu) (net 2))
 (segment (start 70.95 28.6) (end 71.95 28.6) (width 0.254) (layer B.Cu) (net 2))
 (segment (start 69.5 30.05) (end 70.95 28.6) (width 0.254) (layer B.Cu) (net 2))
 (segment (start 68.41 32.6) (end 68.41 31.59) (width 0.254) (layer F.Cu) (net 2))
 (via (at 69.35 30.05) (size 0.889) (layers F.Cu B.Cu) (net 2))
 (segment (start 68.41 31.59) (end 69.35 30.65) (width 0.254) (layer F.Cu) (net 2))
 (segment (start 69.35 30.65) (end 69.35 30.05) (width 0.254) (layer F.Cu) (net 2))
 (segment (start 74.4525 25.9975) (end 75.13 25.9975) (width 0.254) (layer B.Cu) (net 2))
 (segment (start 73.5 27.05) (end 73.5 26.95) (width 0.254) (layer B.Cu) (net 2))
 (segment (start 73.5 26.95) (end 74.4525 25.9975) (width 0.254) (layer B.Cu) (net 2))
 (segment (start 44.55 32.4) (end 68.21 32.4) (width 0.254) (layer F.Cu) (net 2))
 (segment (start 68.21 32.4) (end 68.41 32.6) (width 0.254) (layer F.Cu) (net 2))
 (segment (start 24.8 25.28) (end 27.23 25.28) (width 0.254) (layer F.Cu) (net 2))
 (segment (start 44.35 32.6) (end 42.54 32.6) (width 0.254) (layer B.Cu) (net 2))
 (segment (start 44.55 32.4) (end 44.35 32.6) (width 0.254) (layer B.Cu) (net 2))
 (via (at 44.55 32.4) (size 0.889) (layers F.Cu B.Cu) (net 2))
 (segment (start 32.4 32.4) (end 44.55 32.4) (width 0.254) (layer F.Cu) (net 2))
 (segment (start 28.85 28.85) (end 32.4 32.4) (width 0.254) (layer F.Cu) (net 2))
 (via (at 28.85 28.85) (size 0.889) (layers F.Cu B.Cu) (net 2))
 (segment (start 28.85 26.9) (end 28.85 28.85) (width 0.254) (layer B.Cu) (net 2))
 (segment (start 28.65 26.7) (end 28.85 26.9) (width 0.254) (layer B.Cu) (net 2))
 (via (at 28.65 26.7) (size 0.889) (layers F.Cu B.Cu) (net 2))
 (segment (start 27.23 25.28) (end 28.65 26.7) (width 0.254) (layer F.Cu) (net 2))
 (segment (start 24.8 22.77) (end 24.8 25.28) (width 0.254) (layer F.Cu) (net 2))
 (segment (start 37.46 32.6) (end 31.551 32.6) (width 0.254) (layer B.Cu) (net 7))
 (segment (start 31.551 32.6) (end 30.8 33.351) (width 0.254) (layer B.Cu) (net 7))
 (segment (start 40 32.6) (end 40 31.45) (width 0.254) (layer B.Cu) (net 7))
 (segment (start 37.46 31.14) (end 37.46 32.6) (width 0.254) (layer B.Cu) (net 7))
 (segment (start 37.7 30.9) (end 37.46 31.14) (width 0.254) (layer B.Cu) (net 7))
 (segment (start 39.45 30.9) (end 37.7 30.9) (width 0.254) (layer B.Cu) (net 7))
 (segment (start 40 31.45) (end 39.45 30.9) (width 0.254) (layer B.Cu) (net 7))
 (segment (start 80.499 26) (end 80.499 29.248) (width 0.254) (layer B.Cu) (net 5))
 (segment (start 80.499 29.248) (end 80.5 29.249) (width 0.254) (layer B.Cu) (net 5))
 (segment (start 77.67 25.9975) (end 80.4965 25.9975) (width 0.254) (layer B.Cu) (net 5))
 (segment (start 80.4965 25.9975) (end 80.499 26) (width 0.254) (layer B.Cu) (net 5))
 (segment (start 70.95 32.6) (end 70.95 31.3) (width 0.254) (layer F.Cu) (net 9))
 (segment (start 73.49 31.44) (end 73.49 32.6) (width 0.254) (layer F.Cu) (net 9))
 (segment (start 73.05 31) (end 73.49 31.44) (width 0.254) (layer F.Cu) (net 9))
 (segment (start 71.25 31) (end 73.05 31) (width 0.254) (layer F.Cu) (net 9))
 (segment (start 70.95 31.3) (end 71.25 31) (width 0.254) (layer F.Cu) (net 9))
 (segment (start 73.49 32.6) (end 79.299 32.6) (width 0.254) (layer F.Cu) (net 9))
 (segment (start 79.299 32.6) (end 79.6 32.901) (width 0.254) (layer F.Cu) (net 9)))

